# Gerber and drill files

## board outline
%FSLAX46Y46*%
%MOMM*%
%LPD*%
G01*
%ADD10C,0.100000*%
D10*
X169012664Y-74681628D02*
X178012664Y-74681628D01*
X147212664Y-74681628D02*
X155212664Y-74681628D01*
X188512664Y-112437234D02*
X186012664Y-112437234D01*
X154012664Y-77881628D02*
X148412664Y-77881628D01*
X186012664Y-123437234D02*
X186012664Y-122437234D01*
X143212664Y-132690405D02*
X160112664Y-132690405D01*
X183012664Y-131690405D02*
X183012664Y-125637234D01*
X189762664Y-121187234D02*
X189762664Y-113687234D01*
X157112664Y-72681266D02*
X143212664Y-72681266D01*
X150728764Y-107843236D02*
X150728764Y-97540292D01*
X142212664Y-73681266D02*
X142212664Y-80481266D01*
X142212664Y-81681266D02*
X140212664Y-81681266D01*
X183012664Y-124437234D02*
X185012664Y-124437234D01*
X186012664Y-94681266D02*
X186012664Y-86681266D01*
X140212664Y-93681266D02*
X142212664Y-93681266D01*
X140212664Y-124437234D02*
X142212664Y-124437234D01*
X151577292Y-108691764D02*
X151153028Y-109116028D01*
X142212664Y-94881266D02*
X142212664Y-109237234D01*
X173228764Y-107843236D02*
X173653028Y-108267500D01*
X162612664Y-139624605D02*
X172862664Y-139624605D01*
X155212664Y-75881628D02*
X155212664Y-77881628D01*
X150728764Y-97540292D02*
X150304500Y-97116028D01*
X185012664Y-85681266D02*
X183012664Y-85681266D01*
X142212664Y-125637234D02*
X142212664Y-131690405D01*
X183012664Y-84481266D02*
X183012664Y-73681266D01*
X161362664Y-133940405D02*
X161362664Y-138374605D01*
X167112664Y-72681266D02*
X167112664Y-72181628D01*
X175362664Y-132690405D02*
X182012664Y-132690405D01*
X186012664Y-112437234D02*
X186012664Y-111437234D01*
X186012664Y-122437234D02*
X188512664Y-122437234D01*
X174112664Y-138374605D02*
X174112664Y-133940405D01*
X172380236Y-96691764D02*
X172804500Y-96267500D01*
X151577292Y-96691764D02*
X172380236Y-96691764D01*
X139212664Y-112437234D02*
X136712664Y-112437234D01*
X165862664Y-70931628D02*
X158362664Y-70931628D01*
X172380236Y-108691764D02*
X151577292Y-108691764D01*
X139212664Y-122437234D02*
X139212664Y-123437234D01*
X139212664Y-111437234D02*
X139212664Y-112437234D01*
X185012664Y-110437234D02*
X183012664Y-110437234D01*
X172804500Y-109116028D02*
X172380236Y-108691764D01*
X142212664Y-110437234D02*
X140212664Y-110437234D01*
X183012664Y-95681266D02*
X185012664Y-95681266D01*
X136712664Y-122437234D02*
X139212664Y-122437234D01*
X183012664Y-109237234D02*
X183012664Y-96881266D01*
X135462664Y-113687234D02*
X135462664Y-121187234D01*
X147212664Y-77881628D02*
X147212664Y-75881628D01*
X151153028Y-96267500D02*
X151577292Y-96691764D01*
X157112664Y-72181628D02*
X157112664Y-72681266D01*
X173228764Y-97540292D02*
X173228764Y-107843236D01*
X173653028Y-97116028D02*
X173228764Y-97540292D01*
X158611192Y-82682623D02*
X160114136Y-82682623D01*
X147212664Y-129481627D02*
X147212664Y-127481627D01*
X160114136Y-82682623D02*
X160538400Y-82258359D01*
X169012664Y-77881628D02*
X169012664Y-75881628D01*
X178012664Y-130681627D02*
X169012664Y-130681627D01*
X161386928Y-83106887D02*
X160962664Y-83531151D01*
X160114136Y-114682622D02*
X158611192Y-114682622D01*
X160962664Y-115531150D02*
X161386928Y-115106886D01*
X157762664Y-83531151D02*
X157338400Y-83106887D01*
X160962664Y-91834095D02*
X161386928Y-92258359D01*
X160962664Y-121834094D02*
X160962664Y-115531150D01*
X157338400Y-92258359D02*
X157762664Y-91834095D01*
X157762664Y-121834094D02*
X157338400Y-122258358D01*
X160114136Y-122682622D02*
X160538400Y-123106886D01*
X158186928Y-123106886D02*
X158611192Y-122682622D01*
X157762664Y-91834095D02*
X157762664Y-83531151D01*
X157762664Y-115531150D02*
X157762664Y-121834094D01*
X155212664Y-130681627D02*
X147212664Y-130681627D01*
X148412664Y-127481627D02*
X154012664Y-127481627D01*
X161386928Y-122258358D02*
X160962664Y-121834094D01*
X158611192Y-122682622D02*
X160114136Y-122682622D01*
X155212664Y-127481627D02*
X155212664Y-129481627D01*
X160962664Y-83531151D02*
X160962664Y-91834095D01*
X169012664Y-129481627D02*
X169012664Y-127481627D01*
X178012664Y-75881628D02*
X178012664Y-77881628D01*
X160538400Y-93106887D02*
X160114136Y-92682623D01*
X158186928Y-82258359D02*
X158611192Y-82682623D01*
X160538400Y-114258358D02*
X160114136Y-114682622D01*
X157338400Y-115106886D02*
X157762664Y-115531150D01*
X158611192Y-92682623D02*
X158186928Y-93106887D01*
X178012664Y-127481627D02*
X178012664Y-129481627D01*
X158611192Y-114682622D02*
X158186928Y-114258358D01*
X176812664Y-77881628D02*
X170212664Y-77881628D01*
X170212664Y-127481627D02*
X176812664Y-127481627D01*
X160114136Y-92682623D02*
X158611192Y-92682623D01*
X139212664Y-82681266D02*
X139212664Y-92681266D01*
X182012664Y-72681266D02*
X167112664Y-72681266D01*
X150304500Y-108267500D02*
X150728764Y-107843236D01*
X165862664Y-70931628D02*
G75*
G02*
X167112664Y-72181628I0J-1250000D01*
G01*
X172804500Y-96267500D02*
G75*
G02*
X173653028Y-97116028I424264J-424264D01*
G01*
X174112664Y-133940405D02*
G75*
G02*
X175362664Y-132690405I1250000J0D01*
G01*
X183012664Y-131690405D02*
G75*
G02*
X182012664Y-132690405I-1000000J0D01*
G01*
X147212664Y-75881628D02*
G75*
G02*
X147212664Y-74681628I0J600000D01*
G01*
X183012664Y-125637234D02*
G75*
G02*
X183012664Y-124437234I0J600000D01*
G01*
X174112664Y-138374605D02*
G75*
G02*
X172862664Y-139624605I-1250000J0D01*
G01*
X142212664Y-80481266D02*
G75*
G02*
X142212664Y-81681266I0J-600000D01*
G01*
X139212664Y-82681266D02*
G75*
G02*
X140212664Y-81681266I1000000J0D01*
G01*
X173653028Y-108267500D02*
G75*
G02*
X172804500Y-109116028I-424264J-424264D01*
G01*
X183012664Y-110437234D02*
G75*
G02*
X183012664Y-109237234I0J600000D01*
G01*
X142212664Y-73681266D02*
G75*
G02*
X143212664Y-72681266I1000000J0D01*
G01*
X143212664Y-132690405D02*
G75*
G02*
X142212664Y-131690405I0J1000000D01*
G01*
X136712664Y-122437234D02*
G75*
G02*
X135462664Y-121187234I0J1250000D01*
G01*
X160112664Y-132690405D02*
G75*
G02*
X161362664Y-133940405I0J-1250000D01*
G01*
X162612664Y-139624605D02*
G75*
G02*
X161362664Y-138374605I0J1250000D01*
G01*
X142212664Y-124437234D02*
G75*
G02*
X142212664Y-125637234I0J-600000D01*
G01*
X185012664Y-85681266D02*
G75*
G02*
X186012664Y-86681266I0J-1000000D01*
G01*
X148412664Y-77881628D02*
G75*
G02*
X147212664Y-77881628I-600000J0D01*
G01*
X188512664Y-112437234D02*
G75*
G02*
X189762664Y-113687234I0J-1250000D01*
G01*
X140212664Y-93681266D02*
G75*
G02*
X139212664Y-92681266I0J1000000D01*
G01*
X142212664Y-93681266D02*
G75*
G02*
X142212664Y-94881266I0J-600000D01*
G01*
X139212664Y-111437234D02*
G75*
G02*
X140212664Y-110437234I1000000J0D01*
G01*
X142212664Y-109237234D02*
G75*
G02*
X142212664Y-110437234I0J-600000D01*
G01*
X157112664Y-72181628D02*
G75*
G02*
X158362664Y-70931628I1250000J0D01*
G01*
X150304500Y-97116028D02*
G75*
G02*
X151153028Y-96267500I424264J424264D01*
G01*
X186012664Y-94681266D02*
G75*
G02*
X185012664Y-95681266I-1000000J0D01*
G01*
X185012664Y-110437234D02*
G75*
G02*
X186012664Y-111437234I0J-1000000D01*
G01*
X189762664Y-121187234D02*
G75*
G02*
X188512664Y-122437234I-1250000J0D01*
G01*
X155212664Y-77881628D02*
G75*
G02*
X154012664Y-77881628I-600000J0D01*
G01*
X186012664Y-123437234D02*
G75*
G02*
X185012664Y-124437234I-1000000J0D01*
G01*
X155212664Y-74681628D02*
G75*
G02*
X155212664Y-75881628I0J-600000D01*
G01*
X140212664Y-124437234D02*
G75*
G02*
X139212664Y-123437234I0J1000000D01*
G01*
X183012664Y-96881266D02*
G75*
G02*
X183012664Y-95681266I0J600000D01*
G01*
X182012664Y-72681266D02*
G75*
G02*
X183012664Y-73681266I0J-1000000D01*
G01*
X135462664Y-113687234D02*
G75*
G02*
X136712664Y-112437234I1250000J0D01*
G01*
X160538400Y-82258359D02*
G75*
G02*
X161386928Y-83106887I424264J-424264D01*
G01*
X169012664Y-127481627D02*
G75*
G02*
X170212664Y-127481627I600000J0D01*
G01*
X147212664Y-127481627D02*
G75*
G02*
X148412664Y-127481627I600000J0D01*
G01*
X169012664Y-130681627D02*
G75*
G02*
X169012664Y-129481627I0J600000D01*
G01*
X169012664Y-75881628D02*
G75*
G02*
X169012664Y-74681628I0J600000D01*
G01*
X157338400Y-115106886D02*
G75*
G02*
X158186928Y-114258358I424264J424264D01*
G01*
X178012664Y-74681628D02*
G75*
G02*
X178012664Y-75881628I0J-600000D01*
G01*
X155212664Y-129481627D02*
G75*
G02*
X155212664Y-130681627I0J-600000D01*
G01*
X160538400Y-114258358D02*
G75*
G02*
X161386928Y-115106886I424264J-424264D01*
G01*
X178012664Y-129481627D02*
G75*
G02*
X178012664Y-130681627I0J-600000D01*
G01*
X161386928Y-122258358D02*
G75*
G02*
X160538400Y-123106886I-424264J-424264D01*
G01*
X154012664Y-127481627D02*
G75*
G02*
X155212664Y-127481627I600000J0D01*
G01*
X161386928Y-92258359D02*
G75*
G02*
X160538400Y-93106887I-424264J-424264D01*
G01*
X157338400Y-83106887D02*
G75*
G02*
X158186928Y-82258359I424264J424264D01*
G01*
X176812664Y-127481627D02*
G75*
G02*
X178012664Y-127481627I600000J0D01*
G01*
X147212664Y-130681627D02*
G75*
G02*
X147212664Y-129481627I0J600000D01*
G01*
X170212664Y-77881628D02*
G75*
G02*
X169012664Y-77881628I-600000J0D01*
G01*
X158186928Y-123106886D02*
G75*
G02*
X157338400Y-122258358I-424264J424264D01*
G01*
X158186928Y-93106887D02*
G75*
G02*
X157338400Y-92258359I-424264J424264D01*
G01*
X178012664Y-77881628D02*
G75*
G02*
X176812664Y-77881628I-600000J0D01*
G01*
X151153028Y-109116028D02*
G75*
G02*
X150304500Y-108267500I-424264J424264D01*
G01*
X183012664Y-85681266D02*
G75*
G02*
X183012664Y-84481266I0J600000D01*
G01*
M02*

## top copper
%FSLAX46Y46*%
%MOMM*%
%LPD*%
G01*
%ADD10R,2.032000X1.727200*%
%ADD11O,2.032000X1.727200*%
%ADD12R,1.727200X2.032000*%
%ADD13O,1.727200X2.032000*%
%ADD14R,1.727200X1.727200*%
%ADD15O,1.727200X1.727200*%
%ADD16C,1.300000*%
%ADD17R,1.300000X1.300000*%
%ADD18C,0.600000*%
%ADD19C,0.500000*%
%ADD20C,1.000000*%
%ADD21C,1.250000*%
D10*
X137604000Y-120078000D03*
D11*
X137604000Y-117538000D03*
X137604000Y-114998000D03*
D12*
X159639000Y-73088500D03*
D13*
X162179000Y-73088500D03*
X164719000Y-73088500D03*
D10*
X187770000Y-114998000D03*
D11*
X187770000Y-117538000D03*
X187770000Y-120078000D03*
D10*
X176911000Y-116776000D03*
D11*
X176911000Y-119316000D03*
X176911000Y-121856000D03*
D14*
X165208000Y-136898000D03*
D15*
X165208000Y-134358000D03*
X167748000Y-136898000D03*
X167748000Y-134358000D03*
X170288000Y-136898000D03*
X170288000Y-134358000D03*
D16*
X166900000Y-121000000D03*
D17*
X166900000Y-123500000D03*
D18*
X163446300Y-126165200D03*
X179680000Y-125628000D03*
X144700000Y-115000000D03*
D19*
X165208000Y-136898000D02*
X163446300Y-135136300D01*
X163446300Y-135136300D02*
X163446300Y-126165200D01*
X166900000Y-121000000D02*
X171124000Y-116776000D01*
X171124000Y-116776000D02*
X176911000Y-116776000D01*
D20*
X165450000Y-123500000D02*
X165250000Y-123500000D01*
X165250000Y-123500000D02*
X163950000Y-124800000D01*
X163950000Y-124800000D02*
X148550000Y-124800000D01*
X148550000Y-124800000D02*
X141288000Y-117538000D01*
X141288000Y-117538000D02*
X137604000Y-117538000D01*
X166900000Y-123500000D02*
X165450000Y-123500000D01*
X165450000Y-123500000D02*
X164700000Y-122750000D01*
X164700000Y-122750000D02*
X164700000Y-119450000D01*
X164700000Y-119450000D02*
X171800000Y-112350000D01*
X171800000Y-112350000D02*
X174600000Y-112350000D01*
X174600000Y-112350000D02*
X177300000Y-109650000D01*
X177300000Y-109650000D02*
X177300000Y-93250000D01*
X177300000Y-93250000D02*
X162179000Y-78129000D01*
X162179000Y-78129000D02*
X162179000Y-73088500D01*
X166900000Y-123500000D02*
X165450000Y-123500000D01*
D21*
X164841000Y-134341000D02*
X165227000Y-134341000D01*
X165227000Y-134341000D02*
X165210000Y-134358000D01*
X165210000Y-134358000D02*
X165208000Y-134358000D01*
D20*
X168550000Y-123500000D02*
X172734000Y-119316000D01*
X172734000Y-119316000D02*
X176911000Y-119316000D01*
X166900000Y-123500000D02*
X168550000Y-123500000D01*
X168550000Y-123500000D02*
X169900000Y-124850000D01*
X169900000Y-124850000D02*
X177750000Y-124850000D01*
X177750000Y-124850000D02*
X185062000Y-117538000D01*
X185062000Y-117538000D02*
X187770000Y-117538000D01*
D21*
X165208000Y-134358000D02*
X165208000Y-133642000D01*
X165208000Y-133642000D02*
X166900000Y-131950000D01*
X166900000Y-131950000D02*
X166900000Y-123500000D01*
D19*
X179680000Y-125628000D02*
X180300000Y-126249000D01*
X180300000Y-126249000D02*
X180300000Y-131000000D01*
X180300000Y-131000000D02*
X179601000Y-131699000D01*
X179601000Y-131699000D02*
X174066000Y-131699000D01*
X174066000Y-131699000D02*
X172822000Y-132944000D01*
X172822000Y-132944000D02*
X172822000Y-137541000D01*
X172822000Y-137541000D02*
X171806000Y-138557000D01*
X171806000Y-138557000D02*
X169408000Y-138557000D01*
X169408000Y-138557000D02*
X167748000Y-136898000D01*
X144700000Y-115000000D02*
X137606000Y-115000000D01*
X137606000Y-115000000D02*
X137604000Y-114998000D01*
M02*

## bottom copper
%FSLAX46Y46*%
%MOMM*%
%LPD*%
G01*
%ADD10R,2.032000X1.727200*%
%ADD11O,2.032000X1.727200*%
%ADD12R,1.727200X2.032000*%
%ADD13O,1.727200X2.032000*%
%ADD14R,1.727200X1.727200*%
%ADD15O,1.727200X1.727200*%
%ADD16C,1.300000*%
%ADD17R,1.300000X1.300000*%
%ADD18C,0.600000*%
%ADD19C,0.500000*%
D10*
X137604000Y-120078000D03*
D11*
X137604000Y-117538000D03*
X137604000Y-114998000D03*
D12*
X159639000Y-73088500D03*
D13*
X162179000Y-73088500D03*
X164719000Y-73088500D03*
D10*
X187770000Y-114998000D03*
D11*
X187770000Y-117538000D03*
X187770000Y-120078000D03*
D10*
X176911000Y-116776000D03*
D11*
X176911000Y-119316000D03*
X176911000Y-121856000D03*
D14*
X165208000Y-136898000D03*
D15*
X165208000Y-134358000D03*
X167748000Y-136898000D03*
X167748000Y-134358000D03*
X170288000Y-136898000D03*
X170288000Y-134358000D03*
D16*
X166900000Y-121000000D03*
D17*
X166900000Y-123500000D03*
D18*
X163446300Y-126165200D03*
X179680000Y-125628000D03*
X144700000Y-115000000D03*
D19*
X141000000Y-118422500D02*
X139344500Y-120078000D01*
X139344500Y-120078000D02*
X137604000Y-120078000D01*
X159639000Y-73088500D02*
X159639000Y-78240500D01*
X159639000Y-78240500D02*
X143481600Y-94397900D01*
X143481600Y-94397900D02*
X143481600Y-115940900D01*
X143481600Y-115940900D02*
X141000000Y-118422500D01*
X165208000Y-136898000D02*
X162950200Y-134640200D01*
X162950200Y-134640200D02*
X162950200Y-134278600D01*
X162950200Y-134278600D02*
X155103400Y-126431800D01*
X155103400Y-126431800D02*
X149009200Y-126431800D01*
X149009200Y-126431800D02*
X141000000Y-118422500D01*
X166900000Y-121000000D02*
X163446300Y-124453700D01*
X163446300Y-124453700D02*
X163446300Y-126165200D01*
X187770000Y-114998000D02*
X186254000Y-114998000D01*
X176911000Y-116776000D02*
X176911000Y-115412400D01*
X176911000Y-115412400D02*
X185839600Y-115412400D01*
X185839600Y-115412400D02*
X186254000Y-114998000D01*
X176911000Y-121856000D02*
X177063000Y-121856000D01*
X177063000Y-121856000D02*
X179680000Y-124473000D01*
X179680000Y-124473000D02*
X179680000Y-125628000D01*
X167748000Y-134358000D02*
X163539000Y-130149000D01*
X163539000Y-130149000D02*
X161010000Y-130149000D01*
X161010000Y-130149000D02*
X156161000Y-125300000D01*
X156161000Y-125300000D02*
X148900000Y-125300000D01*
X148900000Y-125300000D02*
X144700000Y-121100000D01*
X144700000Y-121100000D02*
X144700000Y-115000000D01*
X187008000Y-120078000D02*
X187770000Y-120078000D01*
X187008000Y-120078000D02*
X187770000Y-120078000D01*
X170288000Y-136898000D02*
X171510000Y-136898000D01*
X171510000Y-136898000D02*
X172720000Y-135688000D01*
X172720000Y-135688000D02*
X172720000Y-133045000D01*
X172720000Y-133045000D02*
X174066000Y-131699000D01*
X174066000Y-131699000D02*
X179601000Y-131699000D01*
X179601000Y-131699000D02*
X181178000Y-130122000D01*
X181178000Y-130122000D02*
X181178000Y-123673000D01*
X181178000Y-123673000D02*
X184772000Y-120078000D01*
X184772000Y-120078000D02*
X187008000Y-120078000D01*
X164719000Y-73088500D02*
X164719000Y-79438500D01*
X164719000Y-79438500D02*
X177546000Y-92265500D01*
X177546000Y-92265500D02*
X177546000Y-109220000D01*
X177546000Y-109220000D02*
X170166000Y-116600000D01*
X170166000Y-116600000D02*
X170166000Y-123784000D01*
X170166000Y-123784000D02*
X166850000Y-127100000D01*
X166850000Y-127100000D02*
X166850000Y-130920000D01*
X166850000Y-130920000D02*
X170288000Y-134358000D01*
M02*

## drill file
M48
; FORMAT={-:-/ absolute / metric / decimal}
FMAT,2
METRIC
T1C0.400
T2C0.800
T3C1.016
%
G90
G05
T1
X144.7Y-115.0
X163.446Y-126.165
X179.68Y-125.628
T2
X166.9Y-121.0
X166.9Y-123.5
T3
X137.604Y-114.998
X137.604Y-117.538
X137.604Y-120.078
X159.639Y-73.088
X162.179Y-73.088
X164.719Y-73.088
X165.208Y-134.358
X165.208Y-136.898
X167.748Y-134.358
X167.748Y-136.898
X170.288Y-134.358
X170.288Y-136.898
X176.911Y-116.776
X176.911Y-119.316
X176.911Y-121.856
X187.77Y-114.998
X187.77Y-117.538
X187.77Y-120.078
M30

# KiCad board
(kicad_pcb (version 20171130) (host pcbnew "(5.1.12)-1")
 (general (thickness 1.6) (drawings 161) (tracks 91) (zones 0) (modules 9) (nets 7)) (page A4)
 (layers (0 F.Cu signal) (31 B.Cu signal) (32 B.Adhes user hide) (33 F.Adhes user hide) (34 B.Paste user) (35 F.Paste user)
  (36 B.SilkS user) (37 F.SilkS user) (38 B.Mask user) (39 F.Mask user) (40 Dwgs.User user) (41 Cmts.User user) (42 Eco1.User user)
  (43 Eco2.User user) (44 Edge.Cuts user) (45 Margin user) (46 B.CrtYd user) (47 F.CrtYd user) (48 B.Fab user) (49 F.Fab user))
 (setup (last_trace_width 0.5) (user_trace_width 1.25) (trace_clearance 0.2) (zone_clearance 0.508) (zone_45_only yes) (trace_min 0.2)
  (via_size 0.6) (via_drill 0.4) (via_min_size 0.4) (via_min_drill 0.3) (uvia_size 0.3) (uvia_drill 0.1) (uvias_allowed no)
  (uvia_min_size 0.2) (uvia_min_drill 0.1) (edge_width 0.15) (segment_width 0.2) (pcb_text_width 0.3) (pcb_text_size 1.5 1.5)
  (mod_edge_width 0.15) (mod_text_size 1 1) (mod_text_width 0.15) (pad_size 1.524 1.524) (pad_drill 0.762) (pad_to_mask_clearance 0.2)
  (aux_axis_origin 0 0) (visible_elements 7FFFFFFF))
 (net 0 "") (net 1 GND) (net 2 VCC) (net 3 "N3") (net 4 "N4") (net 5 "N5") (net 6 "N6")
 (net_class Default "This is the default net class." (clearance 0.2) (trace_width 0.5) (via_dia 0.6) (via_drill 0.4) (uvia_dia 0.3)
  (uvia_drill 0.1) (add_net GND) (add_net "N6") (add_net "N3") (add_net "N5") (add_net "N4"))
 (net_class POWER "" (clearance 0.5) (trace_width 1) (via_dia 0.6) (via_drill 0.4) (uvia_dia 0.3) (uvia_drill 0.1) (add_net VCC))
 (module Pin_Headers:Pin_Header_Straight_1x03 (layer F.Cu) (at 137.604 120.078 180)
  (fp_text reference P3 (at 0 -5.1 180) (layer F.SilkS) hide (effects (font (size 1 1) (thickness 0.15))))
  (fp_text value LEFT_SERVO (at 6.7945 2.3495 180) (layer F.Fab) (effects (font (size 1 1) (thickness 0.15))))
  (pad 1 thru_hole rect (at 0 0 180) (size 2.032 1.7272) (drill 1.016) (layers *.Cu *.Mask F.SilkS) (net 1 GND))
  (pad 2 thru_hole oval (at 0 2.54 180) (size 2.032 1.7272) (drill 1.016) (layers *.Cu *.Mask F.SilkS) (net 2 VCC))
  (pad 3 thru_hole oval (at 0 5.08 180) (size 2.032 1.7272) (drill 1.016) (layers *.Cu *.Mask F.SilkS) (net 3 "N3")))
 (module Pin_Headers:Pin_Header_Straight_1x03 (layer F.Cu) (at 159.639 73.0885 90)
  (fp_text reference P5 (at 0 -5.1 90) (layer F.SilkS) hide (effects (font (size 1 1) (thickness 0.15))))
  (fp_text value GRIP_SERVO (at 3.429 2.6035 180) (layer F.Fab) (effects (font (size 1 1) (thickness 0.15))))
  (pad 1 thru_hole rect (at 0 0 90) (size 2.032 1.7272) (drill 1.016) (layers *.Cu *.Mask F.SilkS) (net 1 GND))
  (pad 2 thru_hole oval (at 0 2.54 90) (size 2.032 1.7272) (drill 1.016) (layers *.Cu *.Mask F.SilkS) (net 2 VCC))
  (pad 3 thru_hole oval (at 0 5.08 90) (size 2.032 1.7272) (drill 1.016) (layers *.Cu *.Mask F.SilkS) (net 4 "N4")))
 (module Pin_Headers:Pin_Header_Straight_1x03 (layer F.Cu) (at 187.77 114.998)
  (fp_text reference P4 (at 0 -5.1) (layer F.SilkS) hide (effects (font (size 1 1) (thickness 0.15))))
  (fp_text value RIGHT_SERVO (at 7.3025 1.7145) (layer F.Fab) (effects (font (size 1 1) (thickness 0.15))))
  (pad 1 thru_hole rect (at 0 0) (size 2.032 1.7272) (drill 1.016) (layers *.Cu *.Mask F.SilkS) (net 1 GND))
  (pad 2 thru_hole oval (at 0 2.54) (size 2.032 1.7272) (drill 1.016) (layers *.Cu *.Mask F.SilkS) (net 2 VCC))
  (pad 3 thru_hole oval (at 0 5.08) (size 2.032 1.7272) (drill 1.016) (layers *.Cu *.Mask F.SilkS) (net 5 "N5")))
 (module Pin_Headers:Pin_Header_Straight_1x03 (layer F.Cu) (at 176.911 116.776)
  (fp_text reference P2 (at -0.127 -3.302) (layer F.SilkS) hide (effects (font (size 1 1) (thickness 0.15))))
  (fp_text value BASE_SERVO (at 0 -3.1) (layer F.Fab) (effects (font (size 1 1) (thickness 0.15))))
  (pad 1 thru_hole rect (at 0 0) (size 2.032 1.7272) (drill 1.016) (layers *.Cu *.Mask F.SilkS) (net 1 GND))
  (pad 2 thru_hole oval (at 0 2.54) (size 2.032 1.7272) (drill 1.016) (layers *.Cu *.Mask F.SilkS) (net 2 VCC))
  (pad 3 thru_hole oval (at 0 5.08) (size 2.032 1.7272) (drill 1.016) (layers *.Cu *.Mask F.SilkS) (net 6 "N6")))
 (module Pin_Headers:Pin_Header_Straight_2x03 (layer F.Cu) (at 165.208 136.898 90)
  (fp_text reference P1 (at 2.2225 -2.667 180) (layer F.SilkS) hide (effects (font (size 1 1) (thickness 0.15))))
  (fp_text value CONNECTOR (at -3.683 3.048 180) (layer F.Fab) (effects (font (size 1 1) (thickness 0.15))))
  (pad 1 thru_hole rect (at 0 0 90) (size 1.7272 1.7272) (drill 1.016) (layers *.Cu *.Mask F.SilkS) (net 1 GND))
  (pad 2 thru_hole oval (at 2.54 0 90) (size 1.7272 1.7272) (drill 1.016) (layers *.Cu *.Mask F.SilkS) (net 2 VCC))
  (pad 3 thru_hole oval (at 0 2.54 90) (size 1.7272 1.7272) (drill 1.016) (layers *.Cu *.Mask F.SilkS) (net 6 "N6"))
  (pad 4 thru_hole oval (at 2.54 2.54 90) (size 1.7272 1.7272) (drill 1.016) (layers *.Cu *.Mask F.SilkS) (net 3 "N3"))
  (pad 5 thru_hole oval (at 0 5.08 90) (size 1.7272 1.7272) (drill 1.016) (layers *.Cu *.Mask F.SilkS) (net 5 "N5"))
  (pad 6 thru_hole oval (at 2.54 5.08 90) (size 1.7272 1.7272) (drill 1.016) (layers *.Cu *.Mask F.SilkS) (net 4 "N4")))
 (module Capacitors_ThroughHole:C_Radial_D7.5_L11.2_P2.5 (layer F.Cu) (at 166.9 123.5 90)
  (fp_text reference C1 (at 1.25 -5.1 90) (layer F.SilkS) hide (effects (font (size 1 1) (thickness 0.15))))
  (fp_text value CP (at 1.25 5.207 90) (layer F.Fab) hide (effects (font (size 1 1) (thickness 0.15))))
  (pad 2 thru_hole circle (at 2.5 0 90) (size 1.3 1.3) (drill 0.8) (layers *.Cu *.Mask F.SilkS) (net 1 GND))
  (pad 1 thru_hole rect (at 0 0 90) (size 1.3 1.3) (drill 0.8) (layers *.Cu *.Mask F.SilkS) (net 2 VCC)))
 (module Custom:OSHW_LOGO (layer B.Cu) (at 150.25 118.5 180)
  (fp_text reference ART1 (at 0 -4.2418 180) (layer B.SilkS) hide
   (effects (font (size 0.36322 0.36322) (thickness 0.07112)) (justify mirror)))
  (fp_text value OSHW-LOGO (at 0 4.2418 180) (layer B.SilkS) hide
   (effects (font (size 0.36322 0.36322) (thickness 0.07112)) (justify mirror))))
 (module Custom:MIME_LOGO (layer B.Cu) (at 171.45 87.249 180)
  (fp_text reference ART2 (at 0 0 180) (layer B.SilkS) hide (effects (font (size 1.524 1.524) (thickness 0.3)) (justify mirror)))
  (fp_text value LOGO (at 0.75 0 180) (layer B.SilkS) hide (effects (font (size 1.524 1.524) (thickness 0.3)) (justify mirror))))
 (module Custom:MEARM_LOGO (layer B.Cu) (at 149.6695 86.868 180)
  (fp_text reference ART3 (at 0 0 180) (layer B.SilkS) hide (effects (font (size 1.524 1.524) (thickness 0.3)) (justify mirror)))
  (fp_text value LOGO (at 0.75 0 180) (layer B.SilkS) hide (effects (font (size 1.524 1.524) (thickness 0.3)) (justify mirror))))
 (gr_line (start 169.012664 74.681628) (end 178.012664 74.681628) (layer Edge.Cuts) (width 0.1))
 (gr_line (start 147.212664 74.681628) (end 155.212664 74.681628) (layer Edge.Cuts) (width 0.1))
 (gr_line (start 188.512664 112.437234) (end 186.012664 112.437234) (layer Edge.Cuts) (width 0.1))
 (gr_line (start 154.012664 77.881628) (end 148.412664 77.881628) (layer Edge.Cuts) (width 0.1))
 (gr_line (start 186.012664 123.437234) (end 186.012664 122.437234) (layer Edge.Cuts) (width 0.1))
 (gr_line (start 143.212664 132.690405) (end 160.112664 132.690405) (layer Edge.Cuts) (width 0.1))
 (gr_line (start 183.012664 131.690405) (end 183.012664 125.637234) (layer Edge.Cuts) (width 0.1))
 (gr_line (start 189.762664 121.187234) (end 189.762664 113.687234) (layer Edge.Cuts) (width 0.1))
 (gr_line (start 157.112664 72.681266) (end 143.212664 72.681266) (layer Edge.Cuts) (width 0.1))
 (gr_line (start 150.728764 107.843236) (end 150.728764 97.540292) (layer Edge.Cuts) (width 0.1))
 (gr_line (start 142.212664 73.681266) (end 142.212664 80.481266) (layer Edge.Cuts) (width 0.1))
 (gr_line (start 142.212664 81.681266) (end 140.212664 81.681266) (layer Edge.Cuts) (width 0.1))
 (gr_line (start 183.012664 124.437234) (end 185.012664 124.437234) (layer Edge.Cuts) (width 0.1))
 (gr_line (start 186.012664 94.681266) (end 186.012664 86.681266) (layer Edge.Cuts) (width 0.1))
 (gr_line (start 140.212664 93.681266) (end 142.212664 93.681266) (layer Edge.Cuts) (width 0.1))
 (gr_line (start 140.212664 124.437234) (end 142.212664 124.437234) (layer Edge.Cuts) (width 0.1))
 (gr_line (start 151.577292 108.691764) (end 151.153028 109.116028) (layer Edge.Cuts) (width 0.1))
 (gr_line (start 142.212664 94.881266) (end 142.212664 109.237234) (layer Edge.Cuts) (width 0.1))
 (gr_line (start 173.228764 107.843236) (end 173.653028 108.2675) (layer Edge.Cuts) (width 0.1))
 (gr_line (start 162.612664 139.624605) (end 172.862664 139.624605) (layer Edge.Cuts) (width 0.1))
 (gr_line (start 155.212664 75.881628) (end 155.212664 77.881628) (layer Edge.Cuts) (width 0.1))
 (gr_line (start 150.728764 97.540292) (end 150.3045 97.116028) (layer Edge.Cuts) (width 0.1))
 (gr_line (start 185.012664 85.681266) (end 183.012664 85.681266) (layer Edge.Cuts) (width 0.1))
 (gr_line (start 142.212664 125.637234) (end 142.212664 131.690405) (layer Edge.Cuts) (width 0.1))
 (gr_line (start 183.012664 84.481266) (end 183.012664 73.681266) (layer Edge.Cuts) (width 0.1))
 (gr_line (start 161.362664 133.940405) (end 161.362664 138.374605) (layer Edge.Cuts) (width 0.1))
 (gr_line (start 167.112664 72.681266) (end 167.112664 72.181628) (layer Edge.Cuts) (width 0.1))
 (gr_line (start 175.362664 132.690405) (end 182.012664 132.690405) (layer Edge.Cuts) (width 0.1))
 (gr_line (start 186.012664 112.437234) (end 186.012664 111.437234) (layer Edge.Cuts) (width 0.1))
 (gr_line (start 186.012664 122.437234) (end 188.512664 122.437234) (layer Edge.Cuts) (width 0.1))
 (gr_line (start 174.112664 138.374605) (end 174.112664 133.940405) (layer Edge.Cuts) (width 0.1))
 (gr_line (start 172.380236 96.691764) (end 172.8045 96.2675) (layer Edge.Cuts) (width 0.1))
 (gr_line (start 151.577292 96.691764) (end 172.380236 96.691764) (layer Edge.Cuts) (width 0.1))
 (gr_line (start 139.212664 112.437234) (end 136.712664 112.437234) (layer Edge.Cuts) (width 0.1))
 (gr_line (start 165.862664 70.931628) (end 158.362664 70.931628) (layer Edge.Cuts) (width 0.1))
 (gr_line (start 172.380236 108.691764) (end 151.577292 108.691764) (layer Edge.Cuts) (width 0.1))
 (gr_line (start 139.212664 122.437234) (end 139.212664 123.437234) (layer Edge.Cuts) (width 0.1))
 (gr_line (start 139.212664 111.437234) (end 139.212664 112.437234) (layer Edge.Cuts) (width 0.1))
 (gr_line (start 185.012664 110.437234) (end 183.012664 110.437234) (layer Edge.Cuts) (width 0.1))
 (gr_line (start 172.8045 109.116028) (end 172.380236 108.691764) (layer Edge.Cuts) (width 0.1))
 (gr_line (start 142.212664 110.437234) (end 140.212664 110.437234) (layer Edge.Cuts) (width 0.1))
 (gr_line (start 183.012664 95.681266) (end 185.012664 95.681266) (layer Edge.Cuts) (width 0.1))
 (gr_line (start 136.712664 122.437234) (end 139.212664 122.437234) (layer Edge.Cuts) (width 0.1))
 (gr_line (start 183.012664 109.237234) (end 183.012664 96.881266) (layer Edge.Cuts) (width 0.1))
 (gr_line (start 135.462664 113.687234) (end 135.462664 121.187234) (layer Edge.Cuts) (width 0.1))
 (gr_line (start 147.212664 77.881628) (end 147.212664 75.881628) (layer Edge.Cuts) (width 0.1))
 (gr_line (start 151.153028 96.2675) (end 151.577292 96.691764) (layer Edge.Cuts) (width 0.1))
 (gr_line (start 157.112664 72.181628) (end 157.112664 72.681266) (layer Edge.Cuts) (width 0.1))
 (gr_line (start 173.228764 97.540292) (end 173.228764 107.843236) (layer Edge.Cuts) (width 0.1))
 (gr_line (start 173.653028 97.116028) (end 173.228764 97.540292) (layer Edge.Cuts) (width 0.1))
 (gr_line (start 158.611192 82.682623) (end 160.114136 82.682623) (layer Edge.Cuts) (width 0.1))
 (gr_line (start 147.212664 129.481627) (end 147.212664 127.481627) (layer Edge.Cuts) (width 0.1))
 (gr_line (start 160.114136 82.682623) (end 160.5384 82.258359) (layer Edge.Cuts) (width 0.1))
 (gr_line (start 169.012664 77.881628) (end 169.012664 75.881628) (layer Edge.Cuts) (width 0.1))
 (gr_line (start 178.012664 130.681627) (end 169.012664 130.681627) (layer Edge.Cuts) (width 0.1))
 (gr_line (start 161.386928 83.106887) (end 160.962664 83.531151) (layer Edge.Cuts) (width 0.1))
 (gr_line (start 160.114136 114.682622) (end 158.611192 114.682622) (layer Edge.Cuts) (width 0.1))
 (gr_line (start 160.962664 115.53115) (end 161.386928 115.106886) (layer Edge.Cuts) (width 0.1))
 (gr_line (start 157.762664 83.531151) (end 157.3384 83.106887) (layer Edge.Cuts) (width 0.1))
 (gr_line (start 160.962664 91.834095) (end 161.386928 92.258359) (layer Edge.Cuts) (width 0.1))
 (gr_line (start 160.962664 121.834094) (end 160.962664 115.53115) (layer Edge.Cuts) (width 0.1))
 (gr_line (start 157.3384 92.258359) (end 157.762664 91.834095) (layer Edge.Cuts) (width 0.1))
 (gr_line (start 157.762664 121.834094) (end 157.3384 122.258358) (layer Edge.Cuts) (width 0.1))
 (gr_line (start 160.114136 122.682622) (end 160.5384 123.106886) (layer Edge.Cuts) (width 0.1))
 (gr_line (start 158.186928 123.106886) (end 158.611192 122.682622) (layer Edge.Cuts) (width 0.1))
 (gr_line (start 157.762664 91.834095) (end 157.762664 83.531151) (layer Edge.Cuts) (width 0.1))
 (gr_line (start 157.762664 115.53115) (end 157.762664 121.834094) (layer Edge.Cuts) (width 0.1))
 (gr_line (start 155.212664 130.681627) (end 147.212664 130.681627) (layer Edge.Cuts) (width 0.1))
 (gr_line (start 148.412664 127.481627) (end 154.012664 127.481627) (layer Edge.Cuts) (width 0.1))
 (gr_line (start 161.386928 122.258358) (end 160.962664 121.834094) (layer Edge.Cuts) (width 0.1))
 (gr_line (start 158.611192 122.682622) (end 160.114136 122.682622) (layer Edge.Cuts) (width 0.1))
 (gr_line (start 155.212664 127.481627) (end 155.212664 129.481627) (layer Edge.Cuts) (width 0.1))
 (gr_line (start 160.962664 83.531151) (end 160.962664 91.834095) (layer Edge.Cuts) (width 0.1))
 (gr_line (start 169.012664 129.481627) (end 169.012664 127.481627) (layer Edge.Cuts) (width 0.1))
 (gr_line (start 178.012664 75.881628) (end 178.012664 77.881628) (layer Edge.Cuts) (width 0.1))
 (gr_line (start 160.5384 93.106887) (end 160.114136 92.682623) (layer Edge.Cuts) (width 0.1))
 (gr_line (start 158.186928 82.258359) (end 158.611192 82.682623) (layer Edge.Cuts) (width 0.1))
 (gr_line (start 160.5384 114.258358) (end 160.114136 114.682622) (layer Edge.Cuts) (width 0.1))
 (gr_line (start 157.3384 115.106886) (end 157.762664 115.53115) (layer Edge.Cuts) (width 0.1))
 (gr_line (start 158.611192 92.682623) (end 158.186928 93.106887) (layer Edge.Cuts) (width 0.1))
 (gr_line (start 178.012664 127.481627) (end 178.012664 129.481627) (layer Edge.Cuts) (width 0.1))
 (gr_line (start 158.611192 114.682622) (end 158.186928 114.258358) (layer Edge.Cuts) (width 0.1))
 (gr_line (start 176.812664 77.881628) (end 170.212664 77.881628) (layer Edge.Cuts) (width 0.1))
 (gr_line (start 170.212664 127.481627) (end 176.812664 127.481627) (layer Edge.Cuts) (width 0.1))
 (gr_line (start 160.114136 92.682623) (end 158.611192 92.682623) (layer Edge.Cuts) (width 0.1))
 (gr_line (start 139.212664 82.681266) (end 139.212664 92.681266) (layer Edge.Cuts) (width 0.1))
 (gr_line (start 182.012664 72.681266) (end 167.112664 72.681266) (layer Edge.Cuts) (width 0.1))
 (gr_line (start 150.3045 108.2675) (end 150.728764 107.843236) (layer Edge.Cuts) (width 0.1))
 (gr_arc (start 165.862664 72.181628) (end 167.112664 72.181628) (angle -90) (layer Edge.Cuts) (width 0.1))
 (gr_arc (start 173.228764 96.691764) (end 173.653028 97.116028) (angle -180) (layer Edge.Cuts) (width 0.1))
 (gr_arc (start 175.362664 133.940405) (end 175.362664 132.690405) (angle -90) (layer Edge.Cuts) (width 0.1))
 (gr_arc (start 182.012664 131.690405) (end 182.012664 132.690405) (angle -90) (layer Edge.Cuts) (width 0.1))
 (gr_arc (start 147.212664 75.281628) (end 147.212664 74.681628) (angle -180) (layer Edge.Cuts) (width 0.1))
 (gr_arc (start 183.012664 125.037234) (end 183.012664 124.437234) (angle -180) (layer Edge.Cuts) (width 0.1))
 (gr_arc (start 172.862664 138.374605) (end 172.862664 139.624605) (angle -90) (layer Edge.Cuts) (width 0.1))
 (gr_arc (start 142.212664 81.081266) (end 142.212664 81.681266) (angle -180) (layer Edge.Cuts) (width 0.1))
 (gr_arc (start 140.212664 82.681266) (end 140.212664 81.681266) (angle -90) (layer Edge.Cuts) (width 0.1))
 (gr_arc (start 173.228764 108.691764) (end 172.8045 109.116028) (angle -180) (layer Edge.Cuts) (width 0.1))
 (gr_arc (start 183.012664 109.837234) (end 183.012664 109.237234) (angle -180) (layer Edge.Cuts) (width 0.1))
 (gr_arc (start 143.212664 73.681266) (end 143.212664 72.681266) (angle -90) (layer Edge.Cuts) (width 0.1))
 (gr_arc (start 143.212664 131.690405) (end 142.212664 131.690405) (angle -90) (layer Edge.Cuts) (width 0.1))
 (gr_arc (start 136.712664 121.187234) (end 135.462664 121.187234) (angle -90) (layer Edge.Cuts) (width 0.1))
 (gr_arc (start 160.112664 133.940405) (end 161.362664 133.940405) (angle -90) (layer Edge.Cuts) (width 0.1))
 (gr_arc (start 162.612664 138.374605) (end 161.362664 138.374605) (angle -90) (layer Edge.Cuts) (width 0.1))
 (gr_arc (start 142.212664 125.037234) (end 142.212664 125.637234) (angle -180) (layer Edge.Cuts) (width 0.1))
 (gr_arc (start 185.012664 86.681266) (end 186.012664 86.681266) (angle -90) (layer Edge.Cuts) (width 0.1))
 (gr_arc (start 147.812664 77.881628) (end 147.212664 77.881628) (angle -180) (layer Edge.Cuts) (width 0.1))
 (gr_arc (start 188.512664 113.687234) (end 189.762664 113.687234) (angle -90) (layer Edge.Cuts) (width 0.1))
 (gr_arc (start 140.212664 92.681266) (end 139.212664 92.681266) (angle -90) (layer Edge.Cuts) (width 0.1))
 (gr_arc (start 142.212664 94.281266) (end 142.212664 94.881266) (angle -180) (layer Edge.Cuts) (width 0.1))
 (gr_arc (start 140.212664 111.437234) (end 140.212664 110.437234) (angle -90) (layer Edge.Cuts) (width 0.1))
 (gr_arc (start 142.212664 109.837234) (end 142.212664 110.437234) (angle -180) (layer Edge.Cuts) (width 0.1))
 (gr_arc (start 158.362664 72.181628) (end 158.362664 70.931628) (angle -90) (layer Edge.Cuts) (width 0.1))
 (gr_arc (start 150.728764 96.691764) (end 151.153028 96.2675) (angle -180) (layer Edge.Cuts) (width 0.1))
 (gr_arc (start 185.012664 94.681266) (end 185.012664 95.681266) (angle -90) (layer Edge.Cuts) (width 0.1))
 (gr_arc (start 185.012664 111.437234) (end 186.012664 111.437234) (angle -90) (layer Edge.Cuts) (width 0.1))
 (gr_arc (start 188.512664 121.187234) (end 188.512664 122.437234) (angle -90) (layer Edge.Cuts) (width 0.1))
 (gr_arc (start 154.612664 77.881628) (end 154.012664 77.881628) (angle -180) (layer Edge.Cuts) (width 0.1))
 (gr_arc (start 185.012664 123.437234) (end 185.012664 124.437234) (angle -90) (layer Edge.Cuts) (width 0.1))
 (gr_arc (start 155.212664 75.281628) (end 155.212664 75.881628) (angle -180) (layer Edge.Cuts) (width 0.1))
 (gr_arc (start 140.212664 123.437234) (end 139.212664 123.437234) (angle -90) (layer Edge.Cuts) (width 0.1))
 (gr_arc (start 183.012664 96.281266) (end 183.012664 95.681266) (angle -180) (layer Edge.Cuts) (width 0.1))
 (gr_arc (start 182.012664 73.681266) (end 183.012664 73.681266) (angle -90) (layer Edge.Cuts) (width 0.1))
 (gr_arc (start 136.712664 113.687234) (end 136.712664 112.437234) (angle -90) (layer Edge.Cuts) (width 0.1))
 (gr_arc (start 160.962664 82.682623) (end 161.386928 83.106887) (angle -180) (layer Edge.Cuts) (width 0.1))
 (gr_arc (start 169.612664 127.481627) (end 170.212664 127.481627) (angle -180) (layer Edge.Cuts) (width 0.1))
 (gr_arc (start 147.812664 127.481627) (end 148.412664 127.481627) (angle -180) (layer Edge.Cuts) (width 0.1))
 (gr_arc (start 169.012664 130.081627) (end 169.012664 129.481627) (angle -180) (layer Edge.Cuts) (width 0.1))
 (gr_arc (start 169.012664 75.281628) (end 169.012664 74.681628) (angle -180) (layer Edge.Cuts) (width 0.1))
 (gr_arc (start 157.762664 114.682622) (end 158.186928 114.258358) (angle -180) (layer Edge.Cuts) (width 0.1))
 (gr_arc (start 178.012664 75.281628) (end 178.012664 75.881628) (angle -180) (layer Edge.Cuts) (width 0.1))
 (gr_arc (start 155.212664 130.081627) (end 155.212664 130.681627) (angle -180) (layer Edge.Cuts) (width 0.1))
 (gr_arc (start 160.962664 114.682622) (end 161.386928 115.106886) (angle -180) (layer Edge.Cuts) (width 0.1))
 (gr_arc (start 178.012664 130.081627) (end 178.012664 130.681627) (angle -180) (layer Edge.Cuts) (width 0.1))
 (gr_arc (start 160.962664 122.682622) (end 160.5384 123.106886) (angle -180) (layer Edge.Cuts) (width 0.1))
 (gr_arc (start 154.612664 127.481627) (end 155.212664 127.481627) (angle -180) (layer Edge.Cuts) (width 0.1))
 (gr_arc (start 160.962664 92.682623) (end 160.5384 93.106887) (angle -180) (layer Edge.Cuts) (width 0.1))
 (gr_arc (start 157.762664 82.682623) (end 158.186928 82.258359) (angle -180) (layer Edge.Cuts) (width 0.1))
 (gr_arc (start 177.412664 127.481627) (end 178.012664 127.481627) (angle -180) (layer Edge.Cuts) (width 0.1))
 (gr_arc (start 147.212664 130.081627) (end 147.212664 129.481627) (angle -180) (layer Edge.Cuts) (width 0.1))
 (gr_arc (start 169.612664 77.881628) (end 169.012664 77.881628) (angle -180) (layer Edge.Cuts) (width 0.1))
 (gr_arc (start 157.762664 122.682622) (end 157.3384 122.258358) (angle -180) (layer Edge.Cuts) (width 0.1))
 (gr_arc (start 157.762664 92.682623) (end 157.3384 92.258359) (angle -180) (layer Edge.Cuts) (width 0.1))
 (gr_arc (start 177.412664 77.881628) (end 176.812664 77.881628) (angle -180) (layer Edge.Cuts) (width 0.1))
 (gr_arc (start 150.728764 108.691764) (end 150.3045 108.2675) (angle -180) (layer Edge.Cuts) (width 0.1))
 (gr_arc (start 183.012664 85.081266) (end 183.012664 84.481266) (angle -180) (layer Edge.Cuts) (width 0.1))
 (segment (start 141 118.4225) (end 139.3445 120.078) (width 0.5) (layer B.Cu) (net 1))
 (segment (start 139.3445 120.078) (end 137.604 120.078) (width 0.5) (layer B.Cu) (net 1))
 (segment (start 159.639 73.0885) (end 159.639 78.2405) (width 0.5) (layer B.Cu) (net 1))
 (segment (start 159.639 78.2405) (end 143.4816 94.3979) (width 0.5) (layer B.Cu) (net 1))
 (segment (start 143.4816 94.3979) (end 143.4816 115.9409) (width 0.5) (layer B.Cu) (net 1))
 (segment (start 143.4816 115.9409) (end 141 118.4225) (width 0.5) (layer B.Cu) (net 1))
 (segment (start 165.208 136.898) (end 162.9502 134.6402) (width 0.5) (layer B.Cu) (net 1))
 (segment (start 162.9502 134.6402) (end 162.9502 134.2786) (width 0.5) (layer B.Cu) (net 1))
 (segment (start 162.9502 134.2786) (end 155.1034 126.4318) (width 0.5) (layer B.Cu) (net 1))
 (segment (start 155.1034 126.4318) (end 149.0092 126.4318) (width 0.5) (layer B.Cu) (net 1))
 (segment (start 149.0092 126.4318) (end 141 118.4225) (width 0.5) (layer B.Cu) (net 1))
 (segment (start 165.208 136.898) (end 163.4463 135.1363) (width 0.5) (layer F.Cu) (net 1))
 (segment (start 163.4463 135.1363) (end 163.4463 126.1652) (width 0.5) (layer F.Cu) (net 1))
 (segment (start 166.9 121) (end 163.4463 124.4537) (width 0.5) (layer B.Cu) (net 1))
 (segment (start 163.4463 124.4537) (end 163.4463 126.1652) (width 0.5) (layer B.Cu) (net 1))
 (segment (start 187.77 114.998) (end 186.254 114.998) (width 0.5) (layer B.Cu) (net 1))
 (segment (start 176.911 116.776) (end 176.911 115.4124) (width 0.5) (layer B.Cu) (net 1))
 (segment (start 176.911 115.4124) (end 185.8396 115.4124) (width 0.5) (layer B.Cu) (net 1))
 (segment (start 185.8396 115.4124) (end 186.254 114.998) (width 0.5) (layer B.Cu) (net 1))
 (segment (start 166.9 121) (end 171.124 116.776) (width 0.5) (layer F.Cu) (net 1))
 (segment (start 171.124 116.776) (end 176.911 116.776) (width 0.5) (layer F.Cu) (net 1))
 (via (at 163.4463 126.1652) (size 0.6) (layers F.Cu B.Cu) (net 1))
 (segment (start 165.45 123.5) (end 165.25 123.5) (width 1) (layer F.Cu) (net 2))
 (segment (start 165.25 123.5) (end 163.95 124.8) (width 1) (layer F.Cu) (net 2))
 (segment (start 163.95 124.8) (end 148.55 124.8) (width 1) (layer F.Cu) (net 2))
 (segment (start 148.55 124.8) (end 141.288 117.538) (width 1) (layer F.Cu) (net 2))
 (segment (start 141.288 117.538) (end 137.604 117.538) (width 1) (layer F.Cu) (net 2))
 (segment (start 166.9 123.5) (end 165.45 123.5) (width 1) (layer F.Cu) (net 2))
 (segment (start 165.45 123.5) (end 164.7 122.75) (width 1) (layer F.Cu) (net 2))
 (segment (start 164.7 122.75) (end 164.7 119.45) (width 1) (layer F.Cu) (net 2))
 (segment (start 164.7 119.45) (end 171.8 112.35) (width 1) (layer F.Cu) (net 2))
 (segment (start 171.8 112.35) (end 174.6 112.35) (width 1) (layer F.Cu) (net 2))
 (segment (start 174.6 112.35) (end 177.3 109.65) (width 1) (layer F.Cu) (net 2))
 (segment (start 177.3 109.65) (end 177.3 93.25) (width 1) (layer F.Cu) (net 2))
 (segment (start 177.3 93.25) (end 162.179 78.129) (width 1) (layer F.Cu) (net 2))
 (segment (start 162.179 78.129) (end 162.179 73.0885) (width 1) (layer F.Cu) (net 2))
 (segment (start 166.9 123.5) (end 165.45 123.5) (width 1) (layer F.Cu) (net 2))
 (segment (start 164.841 134.341) (end 165.227 134.341) (width 1.25) (layer F.Cu) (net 2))
 (segment (start 165.227 134.341) (end 165.21 134.358) (width 1.25) (layer F.Cu) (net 2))
 (segment (start 165.21 134.358) (end 165.208 134.358) (width 1.25) (layer F.Cu) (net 2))
 (segment (start 168.55 123.5) (end 172.734 119.316) (width 1) (layer F.Cu) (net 2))
 (segment (start 172.734 119.316) (end 176.911 119.316) (width 1) (layer F.Cu) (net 2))
 (segment (start 166.9 123.5) (end 168.55 123.5) (width 1) (layer F.Cu) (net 2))
 (segment (start 168.55 123.5) (end 169.9 124.85) (width 1) (layer F.Cu) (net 2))
 (segment (start 169.9 124.85) (end 177.75 124.85) (width 1) (layer F.Cu) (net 2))
 (segment (start 177.75 124.85) (end 185.062 117.538) (width 1) (layer F.Cu) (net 2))
 (segment (start 185.062 117.538) (end 187.77 117.538) (width 1) (layer F.Cu) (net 2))
 (segment (start 165.208 134.358) (end 165.208 133.642) (width 1.25) (layer F.Cu) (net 2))
 (segment (start 165.208 133.642) (end 166.9 131.95) (width 1.25) (layer F.Cu) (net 2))
 (segment (start 166.9 131.95) (end 166.9 123.5) (width 1.25) (layer F.Cu) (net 2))
 (segment (start 176.911 121.856) (end 177.063 121.856) (width 0.5) (layer B.Cu) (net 6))
 (segment (start 177.063 121.856) (end 179.68 124.473) (width 0.5) (layer B.Cu) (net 6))
 (segment (start 179.68 124.473) (end 179.68 125.628) (width 0.5) (layer B.Cu) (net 6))
 (segment (start 179.68 125.628) (end 180.3 126.249) (width 0.5) (layer F.Cu) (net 6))
 (segment (start 180.3 126.249) (end 180.3 131) (width 0.5) (layer F.Cu) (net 6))
 (segment (start 180.3 131) (end 179.601 131.699) (width 0.5) (layer F.Cu) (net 6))
 (segment (start 179.601 131.699) (end 174.066 131.699) (width 0.5) (layer F.Cu) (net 6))
 (segment (start 174.066 131.699) (end 172.822 132.944) (width 0.5) (layer F.Cu) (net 6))
 (segment (start 172.822 132.944) (end 172.822 137.541) (width 0.5) (layer F.Cu) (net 6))
 (segment (start 172.822 137.541) (end 171.806 138.557) (width 0.5) (layer F.Cu) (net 6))
 (segment (start 171.806 138.557) (end 169.408 138.557) (width 0.5) (layer F.Cu) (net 6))
 (segment (start 169.408 138.557) (end 167.748 136.898) (width 0.5) (layer F.Cu) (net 6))
 (via (at 179.68 125.628) (size 0.6) (layers F.Cu B.Cu) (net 6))
 (segment (start 167.748 134.358) (end 163.539 130.149) (width 0.5) (layer B.Cu) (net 3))
 (segment (start 163.539 130.149) (end 161.01 130.149) (width 0.5) (layer B.Cu) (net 3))
 (segment (start 161.01 130.149) (end 156.161 125.3) (width 0.5) (layer B.Cu) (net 3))
 (segment (start 156.161 125.3) (end 148.9 125.3) (width 0.5) (layer B.Cu) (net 3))
 (segment (start 148.9 125.3) (end 144.7 121.1) (width 0.5) (layer B.Cu) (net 3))
 (segment (start 144.7 121.1) (end 144.7 115) (width 0.5) (layer B.Cu) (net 3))
 (segment (start 144.7 115) (end 137.606 115) (width 0.5) (layer F.Cu) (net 3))
 (segment (start 137.606 115) (end 137.604 114.998) (width 0.5) (layer F.Cu) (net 3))
 (via (at 144.7 115) (size 0.6) (layers F.Cu B.Cu) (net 3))
 (segment (start 187.008 120.078) (end 187.77 120.078) (width 0.5) (layer B.Cu) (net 5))
 (segment (start 187.008 120.078) (end 187.77 120.078) (width 0.5) (layer B.Cu) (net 5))
 (segment (start 170.288 136.898) (end 171.51 136.898) (width 0.5) (layer B.Cu) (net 5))
 (segment (start 171.51 136.898) (end 172.72 135.688) (width 0.5) (layer B.Cu) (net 5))
 (segment (start 172.72 135.688) (end 172.72 133.045) (width 0.5) (layer B.Cu) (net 5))
 (segment (start 172.72 133.045) (end 174.066 131.699) (width 0.5) (layer B.Cu) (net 5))
 (segment (start 174.066 131.699) (end 179.601 131.699) (width 0.5) (layer B.Cu) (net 5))
 (segment (start 179.601 131.699) (end 181.178 130.122) (width 0.5) (layer B.Cu) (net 5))
 (segment (start 181.178 130.122) (end 181.178 123.673) (width 0.5) (layer B.Cu) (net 5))
 (segment (start 181.178 123.673) (end 184.772 120.078) (width 0.5) (layer B.Cu) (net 5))
 (segment (start 184.772 120.078) (end 187.008 120.078) (width 0.5) (layer B.Cu) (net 5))
 (segment (start 164.719 73.0885) (end 164.719 79.4385) (width 0.5) (layer B.Cu) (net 4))
 (segment (start 164.719 79.4385) (end 177.546 92.2655) (width 0.5) (layer B.Cu) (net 4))
 (segment (start 177.546 92.2655) (end 177.546 109.22) (width 0.5) (layer B.Cu) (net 4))
 (segment (start 177.546 109.22) (end 170.166 116.6) (width 0.5) (layer B.Cu) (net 4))
 (segment (start 170.166 116.6) (end 170.166 123.784) (width 0.5) (layer B.Cu) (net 4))
 (segment (start 170.166 123.784) (end 166.85 127.1) (width 0.5) (layer B.Cu) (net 4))
 (segment (start 166.85 127.1) (end 166.85 130.92) (width 0.5) (layer B.Cu) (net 4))
 (segment (start 166.85 130.92) (end 170.288 134.358) (width 0.5) (layer B.Cu) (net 4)))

